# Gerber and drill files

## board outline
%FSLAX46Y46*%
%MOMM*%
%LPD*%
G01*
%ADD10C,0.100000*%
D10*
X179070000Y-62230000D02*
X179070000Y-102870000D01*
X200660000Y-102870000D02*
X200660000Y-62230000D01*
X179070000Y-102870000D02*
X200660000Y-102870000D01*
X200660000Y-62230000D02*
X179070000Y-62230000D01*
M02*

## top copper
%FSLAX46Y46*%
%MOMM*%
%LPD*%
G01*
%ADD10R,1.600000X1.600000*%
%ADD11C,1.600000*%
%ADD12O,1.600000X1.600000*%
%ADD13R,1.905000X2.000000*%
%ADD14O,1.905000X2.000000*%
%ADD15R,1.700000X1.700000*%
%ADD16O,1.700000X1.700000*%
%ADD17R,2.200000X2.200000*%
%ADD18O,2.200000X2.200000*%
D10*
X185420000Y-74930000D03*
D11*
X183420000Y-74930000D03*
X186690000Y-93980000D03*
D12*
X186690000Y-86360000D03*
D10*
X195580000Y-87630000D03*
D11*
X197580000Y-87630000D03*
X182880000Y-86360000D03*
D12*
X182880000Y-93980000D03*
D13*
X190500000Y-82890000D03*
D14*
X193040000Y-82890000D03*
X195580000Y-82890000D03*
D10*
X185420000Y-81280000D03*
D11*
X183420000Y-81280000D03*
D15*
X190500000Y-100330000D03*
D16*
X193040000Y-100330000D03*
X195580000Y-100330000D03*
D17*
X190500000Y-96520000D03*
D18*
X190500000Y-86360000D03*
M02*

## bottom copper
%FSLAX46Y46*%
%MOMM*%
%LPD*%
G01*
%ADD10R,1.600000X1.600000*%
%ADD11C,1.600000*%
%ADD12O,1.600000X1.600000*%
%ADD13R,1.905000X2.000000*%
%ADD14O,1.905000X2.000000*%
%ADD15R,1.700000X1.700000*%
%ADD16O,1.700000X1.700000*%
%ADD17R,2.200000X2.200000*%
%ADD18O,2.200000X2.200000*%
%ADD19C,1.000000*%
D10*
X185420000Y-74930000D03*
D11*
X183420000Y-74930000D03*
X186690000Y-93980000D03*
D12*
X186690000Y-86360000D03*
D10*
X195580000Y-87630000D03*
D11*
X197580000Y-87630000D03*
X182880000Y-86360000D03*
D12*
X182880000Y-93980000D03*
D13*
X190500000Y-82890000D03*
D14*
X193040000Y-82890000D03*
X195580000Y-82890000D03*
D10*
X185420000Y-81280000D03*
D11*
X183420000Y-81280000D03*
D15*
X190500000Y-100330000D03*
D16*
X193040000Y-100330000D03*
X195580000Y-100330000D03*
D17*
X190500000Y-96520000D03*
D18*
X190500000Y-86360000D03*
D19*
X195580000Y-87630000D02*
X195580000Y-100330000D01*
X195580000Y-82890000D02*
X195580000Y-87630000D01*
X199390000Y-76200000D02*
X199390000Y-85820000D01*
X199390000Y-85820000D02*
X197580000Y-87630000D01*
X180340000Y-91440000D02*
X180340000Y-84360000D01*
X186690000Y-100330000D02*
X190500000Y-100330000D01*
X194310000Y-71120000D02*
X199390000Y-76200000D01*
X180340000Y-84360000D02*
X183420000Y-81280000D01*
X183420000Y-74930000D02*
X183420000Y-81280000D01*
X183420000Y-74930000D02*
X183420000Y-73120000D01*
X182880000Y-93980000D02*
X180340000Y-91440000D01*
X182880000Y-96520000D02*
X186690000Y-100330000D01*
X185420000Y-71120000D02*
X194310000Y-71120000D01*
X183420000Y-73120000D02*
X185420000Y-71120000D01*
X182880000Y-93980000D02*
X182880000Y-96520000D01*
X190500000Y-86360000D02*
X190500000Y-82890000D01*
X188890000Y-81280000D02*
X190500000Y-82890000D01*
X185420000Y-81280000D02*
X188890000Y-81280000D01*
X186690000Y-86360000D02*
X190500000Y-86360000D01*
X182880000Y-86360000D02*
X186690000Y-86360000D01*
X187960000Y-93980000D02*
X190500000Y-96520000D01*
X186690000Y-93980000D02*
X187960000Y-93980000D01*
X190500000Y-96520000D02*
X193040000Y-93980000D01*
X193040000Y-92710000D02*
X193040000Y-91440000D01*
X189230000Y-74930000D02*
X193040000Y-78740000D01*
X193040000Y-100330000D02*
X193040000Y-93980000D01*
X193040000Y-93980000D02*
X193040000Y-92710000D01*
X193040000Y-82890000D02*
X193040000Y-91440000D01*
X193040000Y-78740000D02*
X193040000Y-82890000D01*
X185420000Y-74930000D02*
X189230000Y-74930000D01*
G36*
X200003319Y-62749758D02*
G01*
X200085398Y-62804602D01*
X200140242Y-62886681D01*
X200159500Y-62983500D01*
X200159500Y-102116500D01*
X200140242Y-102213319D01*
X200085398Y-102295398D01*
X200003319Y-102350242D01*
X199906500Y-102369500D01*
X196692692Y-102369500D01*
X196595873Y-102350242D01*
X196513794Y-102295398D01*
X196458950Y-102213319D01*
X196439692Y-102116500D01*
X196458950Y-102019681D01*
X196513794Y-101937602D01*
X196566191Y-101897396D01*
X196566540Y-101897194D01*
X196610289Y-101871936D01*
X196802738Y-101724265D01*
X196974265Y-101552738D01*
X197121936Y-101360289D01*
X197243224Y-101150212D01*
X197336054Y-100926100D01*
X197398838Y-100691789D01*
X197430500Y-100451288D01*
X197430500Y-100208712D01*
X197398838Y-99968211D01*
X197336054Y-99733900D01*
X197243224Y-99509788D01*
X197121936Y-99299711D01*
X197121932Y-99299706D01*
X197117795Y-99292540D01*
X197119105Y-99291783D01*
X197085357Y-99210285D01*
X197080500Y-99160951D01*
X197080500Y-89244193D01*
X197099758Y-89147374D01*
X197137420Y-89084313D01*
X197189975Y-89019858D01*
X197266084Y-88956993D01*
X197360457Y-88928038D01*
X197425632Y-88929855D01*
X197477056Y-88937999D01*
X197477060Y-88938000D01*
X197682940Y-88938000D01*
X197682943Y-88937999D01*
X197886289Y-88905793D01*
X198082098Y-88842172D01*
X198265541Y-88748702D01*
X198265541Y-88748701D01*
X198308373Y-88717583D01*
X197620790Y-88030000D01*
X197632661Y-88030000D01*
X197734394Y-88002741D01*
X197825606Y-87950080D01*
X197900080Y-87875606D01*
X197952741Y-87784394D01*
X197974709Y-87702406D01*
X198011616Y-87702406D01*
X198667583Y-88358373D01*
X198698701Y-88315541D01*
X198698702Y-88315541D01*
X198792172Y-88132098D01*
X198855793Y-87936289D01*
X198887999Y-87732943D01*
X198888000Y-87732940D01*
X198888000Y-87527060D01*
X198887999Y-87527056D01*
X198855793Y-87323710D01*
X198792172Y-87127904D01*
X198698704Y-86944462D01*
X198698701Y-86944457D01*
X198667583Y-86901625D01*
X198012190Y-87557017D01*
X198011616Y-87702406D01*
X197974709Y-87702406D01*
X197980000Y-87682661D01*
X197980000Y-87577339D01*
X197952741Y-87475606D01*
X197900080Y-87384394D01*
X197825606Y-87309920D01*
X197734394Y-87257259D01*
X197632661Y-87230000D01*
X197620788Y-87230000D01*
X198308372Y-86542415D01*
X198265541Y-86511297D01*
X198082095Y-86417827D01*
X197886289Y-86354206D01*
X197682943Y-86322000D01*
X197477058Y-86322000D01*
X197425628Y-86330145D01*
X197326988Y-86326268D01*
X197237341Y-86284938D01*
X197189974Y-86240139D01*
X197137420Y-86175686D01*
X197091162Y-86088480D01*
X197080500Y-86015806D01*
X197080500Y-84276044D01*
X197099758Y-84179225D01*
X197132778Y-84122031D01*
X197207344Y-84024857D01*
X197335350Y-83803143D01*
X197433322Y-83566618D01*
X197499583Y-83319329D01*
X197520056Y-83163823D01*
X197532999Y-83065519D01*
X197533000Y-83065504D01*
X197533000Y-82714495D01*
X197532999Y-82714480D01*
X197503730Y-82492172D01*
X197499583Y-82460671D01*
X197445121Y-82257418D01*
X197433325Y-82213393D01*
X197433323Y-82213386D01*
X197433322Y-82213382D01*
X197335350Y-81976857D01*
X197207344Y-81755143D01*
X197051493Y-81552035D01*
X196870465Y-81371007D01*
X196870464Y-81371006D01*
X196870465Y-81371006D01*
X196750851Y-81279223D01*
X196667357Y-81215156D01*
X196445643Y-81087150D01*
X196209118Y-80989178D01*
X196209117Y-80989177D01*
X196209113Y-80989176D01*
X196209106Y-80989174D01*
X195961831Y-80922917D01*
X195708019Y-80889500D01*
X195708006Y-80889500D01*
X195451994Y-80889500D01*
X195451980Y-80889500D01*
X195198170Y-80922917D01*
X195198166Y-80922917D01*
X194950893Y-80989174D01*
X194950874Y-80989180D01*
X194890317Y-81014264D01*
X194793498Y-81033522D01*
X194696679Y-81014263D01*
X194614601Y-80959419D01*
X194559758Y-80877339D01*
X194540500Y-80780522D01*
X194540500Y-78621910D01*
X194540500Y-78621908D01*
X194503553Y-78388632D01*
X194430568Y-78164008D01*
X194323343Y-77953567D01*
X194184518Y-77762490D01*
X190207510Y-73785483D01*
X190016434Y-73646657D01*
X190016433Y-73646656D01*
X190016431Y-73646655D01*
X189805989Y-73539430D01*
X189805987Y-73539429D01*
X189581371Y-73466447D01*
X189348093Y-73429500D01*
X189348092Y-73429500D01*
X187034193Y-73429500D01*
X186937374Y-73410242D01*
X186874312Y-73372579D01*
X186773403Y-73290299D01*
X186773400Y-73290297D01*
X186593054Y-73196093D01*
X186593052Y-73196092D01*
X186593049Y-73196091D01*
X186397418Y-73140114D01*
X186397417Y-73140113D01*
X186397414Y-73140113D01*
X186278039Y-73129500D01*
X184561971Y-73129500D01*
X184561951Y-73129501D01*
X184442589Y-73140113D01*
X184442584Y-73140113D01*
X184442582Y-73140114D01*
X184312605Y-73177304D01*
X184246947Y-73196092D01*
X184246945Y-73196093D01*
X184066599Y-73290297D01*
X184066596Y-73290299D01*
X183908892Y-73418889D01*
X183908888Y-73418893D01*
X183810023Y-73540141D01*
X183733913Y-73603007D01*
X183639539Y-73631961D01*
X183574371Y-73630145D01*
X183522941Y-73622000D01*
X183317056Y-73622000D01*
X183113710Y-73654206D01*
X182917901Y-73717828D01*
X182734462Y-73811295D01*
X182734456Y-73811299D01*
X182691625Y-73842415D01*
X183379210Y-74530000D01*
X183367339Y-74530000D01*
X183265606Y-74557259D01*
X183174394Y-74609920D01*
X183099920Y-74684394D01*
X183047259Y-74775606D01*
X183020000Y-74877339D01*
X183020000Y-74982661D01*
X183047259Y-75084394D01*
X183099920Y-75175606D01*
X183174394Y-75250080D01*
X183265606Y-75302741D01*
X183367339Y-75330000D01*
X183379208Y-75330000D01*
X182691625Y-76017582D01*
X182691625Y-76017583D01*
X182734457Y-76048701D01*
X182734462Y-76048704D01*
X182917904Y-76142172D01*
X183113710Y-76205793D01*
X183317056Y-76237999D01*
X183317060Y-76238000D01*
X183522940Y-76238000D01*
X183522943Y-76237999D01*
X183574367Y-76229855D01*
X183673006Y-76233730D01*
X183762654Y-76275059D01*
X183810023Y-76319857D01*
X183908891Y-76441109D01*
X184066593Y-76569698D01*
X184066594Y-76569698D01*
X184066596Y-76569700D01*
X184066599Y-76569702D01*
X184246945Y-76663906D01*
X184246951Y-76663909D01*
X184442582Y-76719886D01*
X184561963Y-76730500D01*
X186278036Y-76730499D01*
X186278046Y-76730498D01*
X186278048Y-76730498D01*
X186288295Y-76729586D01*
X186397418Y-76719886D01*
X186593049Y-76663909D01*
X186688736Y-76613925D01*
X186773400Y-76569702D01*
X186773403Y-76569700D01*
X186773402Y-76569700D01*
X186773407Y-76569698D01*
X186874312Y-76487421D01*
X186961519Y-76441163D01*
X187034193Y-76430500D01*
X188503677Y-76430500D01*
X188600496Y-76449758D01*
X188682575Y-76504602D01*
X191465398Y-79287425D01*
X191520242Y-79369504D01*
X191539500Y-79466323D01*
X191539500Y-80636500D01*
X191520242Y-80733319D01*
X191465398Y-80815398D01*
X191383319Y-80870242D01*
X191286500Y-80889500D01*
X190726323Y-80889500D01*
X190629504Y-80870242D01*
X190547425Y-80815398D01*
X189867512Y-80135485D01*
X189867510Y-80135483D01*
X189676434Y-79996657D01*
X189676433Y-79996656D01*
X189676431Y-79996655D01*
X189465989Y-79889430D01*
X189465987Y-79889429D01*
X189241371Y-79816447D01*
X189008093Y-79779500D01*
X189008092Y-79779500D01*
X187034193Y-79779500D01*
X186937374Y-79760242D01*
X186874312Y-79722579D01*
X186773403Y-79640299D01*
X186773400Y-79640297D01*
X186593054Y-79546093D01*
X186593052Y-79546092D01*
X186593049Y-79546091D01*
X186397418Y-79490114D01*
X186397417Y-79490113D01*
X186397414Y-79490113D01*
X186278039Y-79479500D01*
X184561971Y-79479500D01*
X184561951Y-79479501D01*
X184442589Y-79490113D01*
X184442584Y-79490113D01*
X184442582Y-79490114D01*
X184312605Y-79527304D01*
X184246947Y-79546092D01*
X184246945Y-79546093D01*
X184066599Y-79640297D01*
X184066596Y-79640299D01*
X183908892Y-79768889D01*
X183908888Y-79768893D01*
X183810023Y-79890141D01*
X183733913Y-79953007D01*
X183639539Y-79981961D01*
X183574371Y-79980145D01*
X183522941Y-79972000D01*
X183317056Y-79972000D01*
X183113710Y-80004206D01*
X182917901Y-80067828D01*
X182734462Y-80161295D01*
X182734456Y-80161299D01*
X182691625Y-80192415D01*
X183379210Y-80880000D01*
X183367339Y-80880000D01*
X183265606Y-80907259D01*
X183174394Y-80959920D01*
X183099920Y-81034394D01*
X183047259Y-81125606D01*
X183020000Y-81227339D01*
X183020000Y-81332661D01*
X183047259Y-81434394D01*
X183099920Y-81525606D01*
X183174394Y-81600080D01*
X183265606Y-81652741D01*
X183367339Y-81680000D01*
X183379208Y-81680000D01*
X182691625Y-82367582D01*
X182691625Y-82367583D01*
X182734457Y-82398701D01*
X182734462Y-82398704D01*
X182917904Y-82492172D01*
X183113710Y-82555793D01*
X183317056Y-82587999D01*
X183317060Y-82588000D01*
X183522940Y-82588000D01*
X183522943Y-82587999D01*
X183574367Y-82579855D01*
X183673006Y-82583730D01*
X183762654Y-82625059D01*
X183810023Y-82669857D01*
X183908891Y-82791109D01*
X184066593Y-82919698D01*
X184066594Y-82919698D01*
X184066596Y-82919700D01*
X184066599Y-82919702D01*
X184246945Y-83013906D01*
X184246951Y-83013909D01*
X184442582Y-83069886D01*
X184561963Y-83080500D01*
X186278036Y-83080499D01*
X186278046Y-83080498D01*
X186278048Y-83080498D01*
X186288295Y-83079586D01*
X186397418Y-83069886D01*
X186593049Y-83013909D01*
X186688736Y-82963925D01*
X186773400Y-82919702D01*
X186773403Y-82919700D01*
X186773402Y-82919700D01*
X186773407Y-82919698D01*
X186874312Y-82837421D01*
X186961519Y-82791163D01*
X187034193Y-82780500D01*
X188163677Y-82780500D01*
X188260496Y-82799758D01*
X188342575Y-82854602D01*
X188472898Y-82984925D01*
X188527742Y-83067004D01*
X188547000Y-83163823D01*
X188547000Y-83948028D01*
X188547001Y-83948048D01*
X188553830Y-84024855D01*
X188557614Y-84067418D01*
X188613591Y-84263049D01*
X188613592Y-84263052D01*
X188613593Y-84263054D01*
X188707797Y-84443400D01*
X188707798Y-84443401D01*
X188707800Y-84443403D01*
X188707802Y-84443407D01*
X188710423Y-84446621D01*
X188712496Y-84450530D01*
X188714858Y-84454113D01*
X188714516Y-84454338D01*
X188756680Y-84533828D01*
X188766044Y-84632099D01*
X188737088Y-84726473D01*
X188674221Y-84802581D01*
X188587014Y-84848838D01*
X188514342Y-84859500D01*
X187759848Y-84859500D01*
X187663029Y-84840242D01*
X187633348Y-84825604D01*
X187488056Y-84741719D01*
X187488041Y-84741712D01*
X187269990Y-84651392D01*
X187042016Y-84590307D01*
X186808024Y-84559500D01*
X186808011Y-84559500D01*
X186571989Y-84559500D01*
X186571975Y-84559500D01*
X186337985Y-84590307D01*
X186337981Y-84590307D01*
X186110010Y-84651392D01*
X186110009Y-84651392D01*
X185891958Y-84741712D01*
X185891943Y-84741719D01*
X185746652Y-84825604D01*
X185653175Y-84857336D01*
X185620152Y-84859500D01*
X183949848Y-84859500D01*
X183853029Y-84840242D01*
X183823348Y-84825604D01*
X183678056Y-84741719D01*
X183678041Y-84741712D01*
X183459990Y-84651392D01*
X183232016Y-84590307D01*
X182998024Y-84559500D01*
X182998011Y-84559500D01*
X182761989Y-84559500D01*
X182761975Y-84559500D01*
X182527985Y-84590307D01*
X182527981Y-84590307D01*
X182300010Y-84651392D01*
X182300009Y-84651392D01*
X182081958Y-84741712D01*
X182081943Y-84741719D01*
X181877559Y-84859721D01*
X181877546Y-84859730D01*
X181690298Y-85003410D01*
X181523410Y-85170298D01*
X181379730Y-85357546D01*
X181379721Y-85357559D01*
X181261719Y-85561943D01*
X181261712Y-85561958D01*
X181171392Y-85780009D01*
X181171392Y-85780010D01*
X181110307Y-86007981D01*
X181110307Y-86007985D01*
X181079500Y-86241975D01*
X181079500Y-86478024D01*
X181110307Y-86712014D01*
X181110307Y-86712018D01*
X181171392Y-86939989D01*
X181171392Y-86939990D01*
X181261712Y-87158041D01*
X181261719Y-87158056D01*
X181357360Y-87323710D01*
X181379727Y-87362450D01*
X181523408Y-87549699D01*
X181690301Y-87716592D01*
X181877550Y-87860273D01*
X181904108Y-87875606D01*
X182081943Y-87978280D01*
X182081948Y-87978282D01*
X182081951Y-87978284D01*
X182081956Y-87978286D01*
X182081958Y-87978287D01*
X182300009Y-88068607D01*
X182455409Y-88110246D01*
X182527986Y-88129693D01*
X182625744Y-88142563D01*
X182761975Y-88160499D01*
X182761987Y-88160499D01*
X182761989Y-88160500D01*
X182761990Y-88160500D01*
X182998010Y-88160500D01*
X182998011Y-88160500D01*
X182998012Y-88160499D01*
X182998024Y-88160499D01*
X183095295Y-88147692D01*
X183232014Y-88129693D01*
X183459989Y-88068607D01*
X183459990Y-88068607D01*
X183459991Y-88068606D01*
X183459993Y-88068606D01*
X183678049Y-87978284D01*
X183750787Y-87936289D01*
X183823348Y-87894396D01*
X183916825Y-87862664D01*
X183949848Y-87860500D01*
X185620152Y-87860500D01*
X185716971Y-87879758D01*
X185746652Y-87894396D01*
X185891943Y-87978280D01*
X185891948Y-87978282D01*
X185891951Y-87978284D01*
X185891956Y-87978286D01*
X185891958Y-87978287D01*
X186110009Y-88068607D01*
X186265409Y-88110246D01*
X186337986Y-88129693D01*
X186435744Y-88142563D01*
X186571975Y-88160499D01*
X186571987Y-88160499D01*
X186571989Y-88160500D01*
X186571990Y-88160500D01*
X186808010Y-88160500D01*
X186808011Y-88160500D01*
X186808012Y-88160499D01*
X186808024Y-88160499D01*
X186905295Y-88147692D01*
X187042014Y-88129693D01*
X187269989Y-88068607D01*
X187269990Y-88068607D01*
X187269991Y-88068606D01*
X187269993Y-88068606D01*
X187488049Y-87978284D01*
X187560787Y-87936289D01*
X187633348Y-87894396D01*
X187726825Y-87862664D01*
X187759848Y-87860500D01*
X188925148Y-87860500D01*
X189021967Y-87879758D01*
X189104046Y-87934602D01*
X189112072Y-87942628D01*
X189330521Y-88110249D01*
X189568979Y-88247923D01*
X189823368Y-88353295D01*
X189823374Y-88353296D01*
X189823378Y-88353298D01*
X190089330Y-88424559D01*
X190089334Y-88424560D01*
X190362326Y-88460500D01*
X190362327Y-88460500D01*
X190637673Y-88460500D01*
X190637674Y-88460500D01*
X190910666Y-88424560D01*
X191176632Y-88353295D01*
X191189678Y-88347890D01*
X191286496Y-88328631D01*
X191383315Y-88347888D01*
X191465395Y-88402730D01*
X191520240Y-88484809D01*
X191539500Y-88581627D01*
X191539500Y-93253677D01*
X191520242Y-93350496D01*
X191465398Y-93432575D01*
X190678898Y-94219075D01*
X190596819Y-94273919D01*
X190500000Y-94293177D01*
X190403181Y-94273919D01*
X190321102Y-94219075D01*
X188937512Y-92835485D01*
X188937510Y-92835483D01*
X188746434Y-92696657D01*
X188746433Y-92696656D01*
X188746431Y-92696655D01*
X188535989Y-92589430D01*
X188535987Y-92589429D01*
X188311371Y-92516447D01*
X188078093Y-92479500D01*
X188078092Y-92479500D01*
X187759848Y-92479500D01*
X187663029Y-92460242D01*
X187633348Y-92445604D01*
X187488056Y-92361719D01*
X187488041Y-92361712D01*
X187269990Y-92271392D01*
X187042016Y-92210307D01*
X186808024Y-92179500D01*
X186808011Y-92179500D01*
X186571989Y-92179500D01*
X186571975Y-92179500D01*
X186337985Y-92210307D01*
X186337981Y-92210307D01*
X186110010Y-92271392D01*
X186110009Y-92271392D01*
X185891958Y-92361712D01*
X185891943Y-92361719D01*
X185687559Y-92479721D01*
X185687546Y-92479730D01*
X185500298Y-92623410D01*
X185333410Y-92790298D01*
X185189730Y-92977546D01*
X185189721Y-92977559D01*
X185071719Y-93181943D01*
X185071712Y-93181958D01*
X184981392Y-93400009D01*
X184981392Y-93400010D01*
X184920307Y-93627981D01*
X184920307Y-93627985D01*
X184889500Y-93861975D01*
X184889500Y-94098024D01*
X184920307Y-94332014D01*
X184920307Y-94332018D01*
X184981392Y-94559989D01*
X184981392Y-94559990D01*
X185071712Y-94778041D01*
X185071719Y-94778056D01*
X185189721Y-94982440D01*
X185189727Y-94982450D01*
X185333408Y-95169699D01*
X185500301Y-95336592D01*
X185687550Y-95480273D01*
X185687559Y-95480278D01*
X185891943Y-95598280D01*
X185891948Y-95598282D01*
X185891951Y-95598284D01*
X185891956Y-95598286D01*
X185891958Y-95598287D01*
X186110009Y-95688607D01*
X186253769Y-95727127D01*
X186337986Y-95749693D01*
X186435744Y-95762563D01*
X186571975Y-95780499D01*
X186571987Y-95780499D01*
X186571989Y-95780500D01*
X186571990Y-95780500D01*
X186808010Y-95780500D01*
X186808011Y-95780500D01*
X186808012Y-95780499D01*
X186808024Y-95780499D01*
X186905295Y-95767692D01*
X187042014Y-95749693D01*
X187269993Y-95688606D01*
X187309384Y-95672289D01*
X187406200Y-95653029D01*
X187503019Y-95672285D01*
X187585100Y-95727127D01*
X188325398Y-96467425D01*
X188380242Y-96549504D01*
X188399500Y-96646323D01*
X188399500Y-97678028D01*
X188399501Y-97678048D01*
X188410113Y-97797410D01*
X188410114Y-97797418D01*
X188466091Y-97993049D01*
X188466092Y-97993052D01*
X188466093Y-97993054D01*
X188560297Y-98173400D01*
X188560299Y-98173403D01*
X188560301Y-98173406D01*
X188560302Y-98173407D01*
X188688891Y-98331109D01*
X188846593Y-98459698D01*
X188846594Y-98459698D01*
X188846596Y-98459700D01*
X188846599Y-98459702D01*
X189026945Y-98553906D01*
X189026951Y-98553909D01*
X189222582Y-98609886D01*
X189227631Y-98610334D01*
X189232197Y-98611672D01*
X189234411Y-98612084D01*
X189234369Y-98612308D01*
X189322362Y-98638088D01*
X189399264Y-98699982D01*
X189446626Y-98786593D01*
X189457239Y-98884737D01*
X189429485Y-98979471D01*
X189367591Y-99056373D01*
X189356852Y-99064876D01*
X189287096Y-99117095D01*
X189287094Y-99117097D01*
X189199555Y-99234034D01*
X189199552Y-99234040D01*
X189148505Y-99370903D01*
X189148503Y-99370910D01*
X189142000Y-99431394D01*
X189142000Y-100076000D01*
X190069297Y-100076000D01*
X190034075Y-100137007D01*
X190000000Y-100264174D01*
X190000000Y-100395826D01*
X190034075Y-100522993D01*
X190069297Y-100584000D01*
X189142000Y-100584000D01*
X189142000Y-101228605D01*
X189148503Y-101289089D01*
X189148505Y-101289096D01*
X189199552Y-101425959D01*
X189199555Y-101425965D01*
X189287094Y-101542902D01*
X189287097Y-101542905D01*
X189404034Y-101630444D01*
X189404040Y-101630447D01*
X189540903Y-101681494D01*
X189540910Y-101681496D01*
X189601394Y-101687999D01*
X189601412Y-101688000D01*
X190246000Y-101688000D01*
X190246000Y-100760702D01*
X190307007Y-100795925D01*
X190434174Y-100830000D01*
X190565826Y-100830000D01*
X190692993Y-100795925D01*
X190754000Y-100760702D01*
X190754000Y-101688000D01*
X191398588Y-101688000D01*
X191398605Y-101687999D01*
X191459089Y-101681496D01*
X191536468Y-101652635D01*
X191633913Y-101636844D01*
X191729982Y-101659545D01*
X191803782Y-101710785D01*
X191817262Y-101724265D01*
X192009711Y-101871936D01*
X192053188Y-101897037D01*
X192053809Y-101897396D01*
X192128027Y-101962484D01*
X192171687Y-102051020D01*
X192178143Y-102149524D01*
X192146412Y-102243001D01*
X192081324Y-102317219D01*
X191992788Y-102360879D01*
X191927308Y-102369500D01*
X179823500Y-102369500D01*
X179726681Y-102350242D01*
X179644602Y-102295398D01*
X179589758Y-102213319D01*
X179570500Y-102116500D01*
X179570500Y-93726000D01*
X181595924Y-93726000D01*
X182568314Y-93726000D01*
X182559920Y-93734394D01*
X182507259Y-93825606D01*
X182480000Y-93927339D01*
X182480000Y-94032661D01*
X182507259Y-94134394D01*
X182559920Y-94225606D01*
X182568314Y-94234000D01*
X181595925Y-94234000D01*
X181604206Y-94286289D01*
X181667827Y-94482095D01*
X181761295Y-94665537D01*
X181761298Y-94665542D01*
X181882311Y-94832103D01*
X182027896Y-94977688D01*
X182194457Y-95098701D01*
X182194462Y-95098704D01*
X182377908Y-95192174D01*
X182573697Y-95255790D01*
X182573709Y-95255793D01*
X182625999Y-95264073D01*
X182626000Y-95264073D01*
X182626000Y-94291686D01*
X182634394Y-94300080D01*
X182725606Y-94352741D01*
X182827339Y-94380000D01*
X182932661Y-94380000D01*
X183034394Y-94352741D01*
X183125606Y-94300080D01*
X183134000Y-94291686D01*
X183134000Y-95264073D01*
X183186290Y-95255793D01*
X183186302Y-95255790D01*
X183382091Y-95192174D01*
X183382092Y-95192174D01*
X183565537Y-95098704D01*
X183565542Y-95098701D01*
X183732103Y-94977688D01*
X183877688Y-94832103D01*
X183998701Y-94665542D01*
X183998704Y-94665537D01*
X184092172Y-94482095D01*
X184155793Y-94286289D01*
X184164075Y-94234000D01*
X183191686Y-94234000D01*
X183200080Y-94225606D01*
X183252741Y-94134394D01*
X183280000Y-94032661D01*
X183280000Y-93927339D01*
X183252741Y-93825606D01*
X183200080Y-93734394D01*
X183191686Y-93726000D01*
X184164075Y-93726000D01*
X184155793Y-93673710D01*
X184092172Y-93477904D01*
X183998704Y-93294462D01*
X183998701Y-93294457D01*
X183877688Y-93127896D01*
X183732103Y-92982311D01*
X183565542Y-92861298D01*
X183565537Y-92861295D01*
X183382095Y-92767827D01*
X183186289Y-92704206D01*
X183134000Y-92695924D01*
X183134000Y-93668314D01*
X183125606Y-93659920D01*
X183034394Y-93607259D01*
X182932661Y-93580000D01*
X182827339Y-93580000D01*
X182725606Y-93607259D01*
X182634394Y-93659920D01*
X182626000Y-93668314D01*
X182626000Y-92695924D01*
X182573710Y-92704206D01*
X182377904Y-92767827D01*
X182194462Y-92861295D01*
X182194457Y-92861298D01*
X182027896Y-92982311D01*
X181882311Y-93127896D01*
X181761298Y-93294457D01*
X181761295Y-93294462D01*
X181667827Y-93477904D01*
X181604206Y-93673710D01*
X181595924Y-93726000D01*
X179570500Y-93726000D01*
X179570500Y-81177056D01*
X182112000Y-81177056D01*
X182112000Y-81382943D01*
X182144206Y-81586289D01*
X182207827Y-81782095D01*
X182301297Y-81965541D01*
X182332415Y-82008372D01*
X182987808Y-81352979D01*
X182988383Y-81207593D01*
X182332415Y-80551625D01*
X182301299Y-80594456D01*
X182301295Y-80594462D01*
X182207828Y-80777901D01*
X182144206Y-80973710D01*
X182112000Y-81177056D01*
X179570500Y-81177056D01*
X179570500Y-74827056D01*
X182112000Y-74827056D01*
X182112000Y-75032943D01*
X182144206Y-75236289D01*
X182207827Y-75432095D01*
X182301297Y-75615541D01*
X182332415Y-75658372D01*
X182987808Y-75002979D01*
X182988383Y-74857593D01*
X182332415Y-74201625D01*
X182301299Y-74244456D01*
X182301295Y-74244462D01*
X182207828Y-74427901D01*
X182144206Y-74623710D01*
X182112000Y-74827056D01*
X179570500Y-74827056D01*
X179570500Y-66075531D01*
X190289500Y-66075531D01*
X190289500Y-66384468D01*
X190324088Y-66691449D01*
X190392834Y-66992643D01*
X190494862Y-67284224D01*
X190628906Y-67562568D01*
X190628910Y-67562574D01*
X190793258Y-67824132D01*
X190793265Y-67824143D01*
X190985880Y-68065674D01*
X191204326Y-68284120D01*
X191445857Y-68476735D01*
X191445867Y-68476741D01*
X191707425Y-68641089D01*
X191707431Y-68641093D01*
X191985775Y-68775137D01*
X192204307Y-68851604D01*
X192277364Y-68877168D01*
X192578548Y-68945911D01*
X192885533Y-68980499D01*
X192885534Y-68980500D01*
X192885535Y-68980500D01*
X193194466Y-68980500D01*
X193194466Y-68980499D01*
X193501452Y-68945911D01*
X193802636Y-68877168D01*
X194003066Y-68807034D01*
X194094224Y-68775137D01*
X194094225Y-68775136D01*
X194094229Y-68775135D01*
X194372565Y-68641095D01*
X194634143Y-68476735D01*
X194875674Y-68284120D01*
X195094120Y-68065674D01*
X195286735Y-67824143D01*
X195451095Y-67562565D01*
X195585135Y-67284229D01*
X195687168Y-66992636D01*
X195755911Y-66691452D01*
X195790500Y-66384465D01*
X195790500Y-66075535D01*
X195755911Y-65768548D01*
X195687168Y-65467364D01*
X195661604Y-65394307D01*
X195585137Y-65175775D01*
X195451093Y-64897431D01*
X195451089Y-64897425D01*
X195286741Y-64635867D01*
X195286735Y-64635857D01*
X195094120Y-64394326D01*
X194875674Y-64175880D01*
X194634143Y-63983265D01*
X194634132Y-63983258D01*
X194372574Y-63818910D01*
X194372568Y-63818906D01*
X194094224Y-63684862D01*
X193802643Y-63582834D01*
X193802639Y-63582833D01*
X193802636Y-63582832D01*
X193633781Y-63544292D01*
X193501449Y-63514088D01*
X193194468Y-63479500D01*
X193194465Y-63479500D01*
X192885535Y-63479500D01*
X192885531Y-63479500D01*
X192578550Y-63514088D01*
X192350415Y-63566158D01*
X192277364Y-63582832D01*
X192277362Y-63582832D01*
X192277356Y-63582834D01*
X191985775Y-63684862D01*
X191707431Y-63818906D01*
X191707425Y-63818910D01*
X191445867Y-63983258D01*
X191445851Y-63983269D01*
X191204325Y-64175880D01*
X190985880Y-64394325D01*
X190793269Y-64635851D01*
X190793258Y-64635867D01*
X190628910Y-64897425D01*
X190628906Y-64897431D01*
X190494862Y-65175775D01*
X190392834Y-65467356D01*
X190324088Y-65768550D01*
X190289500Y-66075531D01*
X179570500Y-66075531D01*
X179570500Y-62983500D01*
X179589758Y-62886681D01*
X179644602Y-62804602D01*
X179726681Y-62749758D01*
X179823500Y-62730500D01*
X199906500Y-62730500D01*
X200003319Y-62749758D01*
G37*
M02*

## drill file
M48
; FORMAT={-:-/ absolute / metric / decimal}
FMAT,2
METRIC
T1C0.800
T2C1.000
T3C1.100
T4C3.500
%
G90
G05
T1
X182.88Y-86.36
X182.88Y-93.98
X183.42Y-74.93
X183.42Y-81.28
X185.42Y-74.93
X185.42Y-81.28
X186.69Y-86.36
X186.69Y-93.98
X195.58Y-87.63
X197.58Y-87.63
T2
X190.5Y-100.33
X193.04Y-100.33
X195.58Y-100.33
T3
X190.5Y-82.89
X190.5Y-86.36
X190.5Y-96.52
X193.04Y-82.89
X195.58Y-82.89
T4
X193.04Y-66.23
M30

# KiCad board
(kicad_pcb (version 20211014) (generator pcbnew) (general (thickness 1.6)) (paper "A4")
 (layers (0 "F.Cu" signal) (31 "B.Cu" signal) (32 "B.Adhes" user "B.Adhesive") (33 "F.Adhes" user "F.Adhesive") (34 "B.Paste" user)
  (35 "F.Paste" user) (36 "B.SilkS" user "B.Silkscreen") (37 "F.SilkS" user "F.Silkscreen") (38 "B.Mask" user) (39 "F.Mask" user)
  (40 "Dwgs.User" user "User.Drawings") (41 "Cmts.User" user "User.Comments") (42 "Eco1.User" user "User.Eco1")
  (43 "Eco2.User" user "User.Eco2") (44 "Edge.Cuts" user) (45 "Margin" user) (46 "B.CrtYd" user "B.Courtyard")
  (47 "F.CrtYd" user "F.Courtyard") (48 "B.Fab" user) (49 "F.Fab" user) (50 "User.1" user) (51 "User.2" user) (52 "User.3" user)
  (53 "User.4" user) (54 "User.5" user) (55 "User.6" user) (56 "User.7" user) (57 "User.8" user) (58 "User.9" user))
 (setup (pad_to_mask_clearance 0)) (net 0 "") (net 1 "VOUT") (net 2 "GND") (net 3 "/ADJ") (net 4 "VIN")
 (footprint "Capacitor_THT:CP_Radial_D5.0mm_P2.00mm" (layer "F.Cu") (at 185.42 74.93 180)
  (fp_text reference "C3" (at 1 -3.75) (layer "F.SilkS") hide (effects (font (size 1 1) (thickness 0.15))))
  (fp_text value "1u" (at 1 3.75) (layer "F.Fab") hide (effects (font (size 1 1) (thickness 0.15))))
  (pad "1" thru_hole rect (at 0 0 180) (size 1.6 1.6) (drill 0.8) (layers *.Cu *.Mask) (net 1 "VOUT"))
  (pad "2" thru_hole circle (at 2 0 180) (size 1.6 1.6) (drill 0.8) (layers *.Cu *.Mask) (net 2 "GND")))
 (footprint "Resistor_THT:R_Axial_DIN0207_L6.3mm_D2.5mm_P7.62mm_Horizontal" (layer "F.Cu") (at 186.69 93.98 90)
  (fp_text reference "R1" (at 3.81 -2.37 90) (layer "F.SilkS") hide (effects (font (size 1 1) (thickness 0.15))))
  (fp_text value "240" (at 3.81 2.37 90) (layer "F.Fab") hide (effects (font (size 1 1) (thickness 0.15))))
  (pad "1" thru_hole circle (at 0 0 90) (size 1.6 1.6) (drill 0.8) (layers *.Cu *.Mask) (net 1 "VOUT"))
  (pad "2" thru_hole oval (at 7.62 0 90) (size 1.6 1.6) (drill 0.8) (layers *.Cu *.Mask) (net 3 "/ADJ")))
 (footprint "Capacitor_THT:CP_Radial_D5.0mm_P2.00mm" (layer "F.Cu") (at 195.58 87.63)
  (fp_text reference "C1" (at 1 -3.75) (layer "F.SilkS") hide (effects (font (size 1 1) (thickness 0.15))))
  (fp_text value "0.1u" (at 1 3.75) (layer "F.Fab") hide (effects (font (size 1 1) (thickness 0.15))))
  (pad "1" thru_hole rect (at 0 0) (size 1.6 1.6) (drill 0.8) (layers *.Cu *.Mask) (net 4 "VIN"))
  (pad "2" thru_hole circle (at 2 0) (size 1.6 1.6) (drill 0.8) (layers *.Cu *.Mask) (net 2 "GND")))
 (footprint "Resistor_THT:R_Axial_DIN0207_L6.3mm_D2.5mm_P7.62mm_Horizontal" (layer "F.Cu") (at 182.88 86.36 -90)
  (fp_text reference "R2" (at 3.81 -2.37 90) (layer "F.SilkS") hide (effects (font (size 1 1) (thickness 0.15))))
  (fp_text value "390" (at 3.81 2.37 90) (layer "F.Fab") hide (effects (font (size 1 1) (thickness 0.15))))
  (pad "1" thru_hole circle (at 0 0 270) (size 1.6 1.6) (drill 0.8) (layers *.Cu *.Mask) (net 3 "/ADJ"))
  (pad "2" thru_hole oval (at 7.62 0 270) (size 1.6 1.6) (drill 0.8) (layers *.Cu *.Mask) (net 2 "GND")))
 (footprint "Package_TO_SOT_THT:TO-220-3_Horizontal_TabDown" (layer "F.Cu") (at 190.5 82.89)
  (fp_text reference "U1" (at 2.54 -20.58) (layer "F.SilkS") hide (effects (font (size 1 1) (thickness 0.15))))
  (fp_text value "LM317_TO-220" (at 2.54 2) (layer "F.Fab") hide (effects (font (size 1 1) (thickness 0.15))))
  (pad "" np_thru_hole oval (at 2.54 -16.66) (size 3.5 3.5) (drill 3.5) (layers F&B.Cu *.Mask))
  (pad "1" thru_hole rect (at 0 0) (size 1.905 2) (drill 1.1) (layers *.Cu *.Mask) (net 3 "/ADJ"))
  (pad "2" thru_hole oval (at 2.54 0) (size 1.905 2) (drill 1.1) (layers *.Cu *.Mask) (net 1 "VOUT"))
  (pad "3" thru_hole oval (at 5.08 0) (size 1.905 2) (drill 1.1) (layers *.Cu *.Mask) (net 4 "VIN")))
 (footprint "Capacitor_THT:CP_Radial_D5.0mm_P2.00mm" (layer "F.Cu") (at 185.42 81.28 180)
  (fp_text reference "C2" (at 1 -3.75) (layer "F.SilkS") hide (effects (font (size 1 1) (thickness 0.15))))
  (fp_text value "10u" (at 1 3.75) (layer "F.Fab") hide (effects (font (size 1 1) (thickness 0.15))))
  (pad "1" thru_hole rect (at 0 0 180) (size 1.6 1.6) (drill 0.8) (layers *.Cu *.Mask) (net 3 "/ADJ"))
  (pad "2" thru_hole circle (at 2 0 180) (size 1.6 1.6) (drill 0.8) (layers *.Cu *.Mask) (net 2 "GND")))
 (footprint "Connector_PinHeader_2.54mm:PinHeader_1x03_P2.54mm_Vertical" (layer "F.Cu") (at 190.5 100.33 90)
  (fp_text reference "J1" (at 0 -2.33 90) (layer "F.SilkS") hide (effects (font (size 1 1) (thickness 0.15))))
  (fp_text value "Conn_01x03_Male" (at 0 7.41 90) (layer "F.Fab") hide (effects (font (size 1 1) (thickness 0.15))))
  (pad "1" thru_hole rect (at 0 0 90) (size 1.7 1.7) (drill 1) (layers *.Cu *.Mask) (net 2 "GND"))
  (pad "2" thru_hole oval (at 0 2.54 90) (size 1.7 1.7) (drill 1) (layers *.Cu *.Mask) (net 1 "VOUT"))
  (pad "3" thru_hole oval (at 0 5.08 90) (size 1.7 1.7) (drill 1) (layers *.Cu *.Mask) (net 4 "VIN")))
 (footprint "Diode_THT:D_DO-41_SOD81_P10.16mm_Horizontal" (layer "F.Cu") (at 190.5 96.52 90)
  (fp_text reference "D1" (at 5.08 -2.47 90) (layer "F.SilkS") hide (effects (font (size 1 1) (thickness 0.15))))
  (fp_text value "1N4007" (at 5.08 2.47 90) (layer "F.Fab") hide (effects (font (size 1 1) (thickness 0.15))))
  (pad "1" thru_hole rect (at 0 0 90) (size 2.2 2.2) (drill 1.1) (layers *.Cu *.Mask) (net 1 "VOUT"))
  (pad "2" thru_hole oval (at 10.16 0 90) (size 2.2 2.2) (drill 1.1) (layers *.Cu *.Mask) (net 3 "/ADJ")))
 (gr_line (start 179.07 62.23) (end 179.07 102.87) (layer "Edge.Cuts") (width 0.1))
 (gr_line (start 200.66 102.87) (end 200.66 62.23) (layer "Edge.Cuts") (width 0.1))
 (gr_line (start 179.07 102.87) (end 200.66 102.87) (layer "Edge.Cuts") (width 0.1))
 (gr_line (start 200.66 62.23) (end 179.07 62.23) (layer "Edge.Cuts") (width 0.1))
 (segment (start 195.58 87.63) (end 195.58 100.33) (width 1) (layer "B.Cu") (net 4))
 (segment (start 195.58 82.89) (end 195.58 87.63) (width 1) (layer "B.Cu") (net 4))
 (segment (start 199.39 76.2) (end 199.39 85.82) (width 1) (layer "B.Cu") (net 2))
 (segment (start 199.39 85.82) (end 197.58 87.63) (width 1) (layer "B.Cu") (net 2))
 (segment (start 180.34 91.44) (end 180.34 84.36) (width 1) (layer "B.Cu") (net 2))
 (segment (start 186.69 100.33) (end 190.5 100.33) (width 1) (layer "B.Cu") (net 2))
 (segment (start 194.31 71.12) (end 199.39 76.2) (width 1) (layer "B.Cu") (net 2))
 (segment (start 180.34 84.36) (end 183.42 81.28) (width 1) (layer "B.Cu") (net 2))
 (segment (start 183.42 74.93) (end 183.42 81.28) (width 1) (layer "B.Cu") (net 2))
 (segment (start 183.42 74.93) (end 183.42 73.12) (width 1) (layer "B.Cu") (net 2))
 (segment (start 182.88 93.98) (end 180.34 91.44) (width 1) (layer "B.Cu") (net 2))
 (segment (start 182.88 96.52) (end 186.69 100.33) (width 1) (layer "B.Cu") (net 2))
 (segment (start 185.42 71.12) (end 194.31 71.12) (width 1) (layer "B.Cu") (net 2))
 (segment (start 183.42 73.12) (end 185.42 71.12) (width 1) (layer "B.Cu") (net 2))
 (segment (start 182.88 93.98) (end 182.88 96.52) (width 1) (layer "B.Cu") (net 2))
 (segment (start 190.5 86.36) (end 190.5 82.89) (width 1) (layer "B.Cu") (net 3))
 (segment (start 188.89 81.28) (end 190.5 82.89) (width 1) (layer "B.Cu") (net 3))
 (segment (start 185.42 81.28) (end 188.89 81.28) (width 1) (layer "B.Cu") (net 3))
 (segment (start 186.69 86.36) (end 190.5 86.36) (width 1) (layer "B.Cu") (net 3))
 (segment (start 182.88 86.36) (end 186.69 86.36) (width 1) (layer "B.Cu") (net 3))
 (segment (start 187.96 93.98) (end 190.5 96.52) (width 1) (layer "B.Cu") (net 1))
 (segment (start 186.69 93.98) (end 187.96 93.98) (width 1) (layer "B.Cu") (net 1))
 (segment (start 190.5 96.52) (end 193.04 93.98) (width 1) (layer "B.Cu") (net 1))
 (segment (start 193.04 92.71) (end 193.04 91.44) (width 1) (layer "B.Cu") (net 1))
 (segment (start 189.23 74.93) (end 193.04 78.74) (width 1) (layer "B.Cu") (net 1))
 (segment (start 193.04 100.33) (end 193.04 93.98) (width 1) (layer "B.Cu") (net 1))
 (segment (start 193.04 93.98) (end 193.04 92.71) (width 1) (layer "B.Cu") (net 1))
 (segment (start 193.04 82.89) (end 193.04 91.44) (width 1) (layer "B.Cu") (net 1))
 (segment (start 193.04 78.74) (end 193.04 82.89) (width 1) (layer "B.Cu") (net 1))
 (segment (start 185.42 74.93) (end 189.23 74.93) (width 1) (layer "B.Cu") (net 1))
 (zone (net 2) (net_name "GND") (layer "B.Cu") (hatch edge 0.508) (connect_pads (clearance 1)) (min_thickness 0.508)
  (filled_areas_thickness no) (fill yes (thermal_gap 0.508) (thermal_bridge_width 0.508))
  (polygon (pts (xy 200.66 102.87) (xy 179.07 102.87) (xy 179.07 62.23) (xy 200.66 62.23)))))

